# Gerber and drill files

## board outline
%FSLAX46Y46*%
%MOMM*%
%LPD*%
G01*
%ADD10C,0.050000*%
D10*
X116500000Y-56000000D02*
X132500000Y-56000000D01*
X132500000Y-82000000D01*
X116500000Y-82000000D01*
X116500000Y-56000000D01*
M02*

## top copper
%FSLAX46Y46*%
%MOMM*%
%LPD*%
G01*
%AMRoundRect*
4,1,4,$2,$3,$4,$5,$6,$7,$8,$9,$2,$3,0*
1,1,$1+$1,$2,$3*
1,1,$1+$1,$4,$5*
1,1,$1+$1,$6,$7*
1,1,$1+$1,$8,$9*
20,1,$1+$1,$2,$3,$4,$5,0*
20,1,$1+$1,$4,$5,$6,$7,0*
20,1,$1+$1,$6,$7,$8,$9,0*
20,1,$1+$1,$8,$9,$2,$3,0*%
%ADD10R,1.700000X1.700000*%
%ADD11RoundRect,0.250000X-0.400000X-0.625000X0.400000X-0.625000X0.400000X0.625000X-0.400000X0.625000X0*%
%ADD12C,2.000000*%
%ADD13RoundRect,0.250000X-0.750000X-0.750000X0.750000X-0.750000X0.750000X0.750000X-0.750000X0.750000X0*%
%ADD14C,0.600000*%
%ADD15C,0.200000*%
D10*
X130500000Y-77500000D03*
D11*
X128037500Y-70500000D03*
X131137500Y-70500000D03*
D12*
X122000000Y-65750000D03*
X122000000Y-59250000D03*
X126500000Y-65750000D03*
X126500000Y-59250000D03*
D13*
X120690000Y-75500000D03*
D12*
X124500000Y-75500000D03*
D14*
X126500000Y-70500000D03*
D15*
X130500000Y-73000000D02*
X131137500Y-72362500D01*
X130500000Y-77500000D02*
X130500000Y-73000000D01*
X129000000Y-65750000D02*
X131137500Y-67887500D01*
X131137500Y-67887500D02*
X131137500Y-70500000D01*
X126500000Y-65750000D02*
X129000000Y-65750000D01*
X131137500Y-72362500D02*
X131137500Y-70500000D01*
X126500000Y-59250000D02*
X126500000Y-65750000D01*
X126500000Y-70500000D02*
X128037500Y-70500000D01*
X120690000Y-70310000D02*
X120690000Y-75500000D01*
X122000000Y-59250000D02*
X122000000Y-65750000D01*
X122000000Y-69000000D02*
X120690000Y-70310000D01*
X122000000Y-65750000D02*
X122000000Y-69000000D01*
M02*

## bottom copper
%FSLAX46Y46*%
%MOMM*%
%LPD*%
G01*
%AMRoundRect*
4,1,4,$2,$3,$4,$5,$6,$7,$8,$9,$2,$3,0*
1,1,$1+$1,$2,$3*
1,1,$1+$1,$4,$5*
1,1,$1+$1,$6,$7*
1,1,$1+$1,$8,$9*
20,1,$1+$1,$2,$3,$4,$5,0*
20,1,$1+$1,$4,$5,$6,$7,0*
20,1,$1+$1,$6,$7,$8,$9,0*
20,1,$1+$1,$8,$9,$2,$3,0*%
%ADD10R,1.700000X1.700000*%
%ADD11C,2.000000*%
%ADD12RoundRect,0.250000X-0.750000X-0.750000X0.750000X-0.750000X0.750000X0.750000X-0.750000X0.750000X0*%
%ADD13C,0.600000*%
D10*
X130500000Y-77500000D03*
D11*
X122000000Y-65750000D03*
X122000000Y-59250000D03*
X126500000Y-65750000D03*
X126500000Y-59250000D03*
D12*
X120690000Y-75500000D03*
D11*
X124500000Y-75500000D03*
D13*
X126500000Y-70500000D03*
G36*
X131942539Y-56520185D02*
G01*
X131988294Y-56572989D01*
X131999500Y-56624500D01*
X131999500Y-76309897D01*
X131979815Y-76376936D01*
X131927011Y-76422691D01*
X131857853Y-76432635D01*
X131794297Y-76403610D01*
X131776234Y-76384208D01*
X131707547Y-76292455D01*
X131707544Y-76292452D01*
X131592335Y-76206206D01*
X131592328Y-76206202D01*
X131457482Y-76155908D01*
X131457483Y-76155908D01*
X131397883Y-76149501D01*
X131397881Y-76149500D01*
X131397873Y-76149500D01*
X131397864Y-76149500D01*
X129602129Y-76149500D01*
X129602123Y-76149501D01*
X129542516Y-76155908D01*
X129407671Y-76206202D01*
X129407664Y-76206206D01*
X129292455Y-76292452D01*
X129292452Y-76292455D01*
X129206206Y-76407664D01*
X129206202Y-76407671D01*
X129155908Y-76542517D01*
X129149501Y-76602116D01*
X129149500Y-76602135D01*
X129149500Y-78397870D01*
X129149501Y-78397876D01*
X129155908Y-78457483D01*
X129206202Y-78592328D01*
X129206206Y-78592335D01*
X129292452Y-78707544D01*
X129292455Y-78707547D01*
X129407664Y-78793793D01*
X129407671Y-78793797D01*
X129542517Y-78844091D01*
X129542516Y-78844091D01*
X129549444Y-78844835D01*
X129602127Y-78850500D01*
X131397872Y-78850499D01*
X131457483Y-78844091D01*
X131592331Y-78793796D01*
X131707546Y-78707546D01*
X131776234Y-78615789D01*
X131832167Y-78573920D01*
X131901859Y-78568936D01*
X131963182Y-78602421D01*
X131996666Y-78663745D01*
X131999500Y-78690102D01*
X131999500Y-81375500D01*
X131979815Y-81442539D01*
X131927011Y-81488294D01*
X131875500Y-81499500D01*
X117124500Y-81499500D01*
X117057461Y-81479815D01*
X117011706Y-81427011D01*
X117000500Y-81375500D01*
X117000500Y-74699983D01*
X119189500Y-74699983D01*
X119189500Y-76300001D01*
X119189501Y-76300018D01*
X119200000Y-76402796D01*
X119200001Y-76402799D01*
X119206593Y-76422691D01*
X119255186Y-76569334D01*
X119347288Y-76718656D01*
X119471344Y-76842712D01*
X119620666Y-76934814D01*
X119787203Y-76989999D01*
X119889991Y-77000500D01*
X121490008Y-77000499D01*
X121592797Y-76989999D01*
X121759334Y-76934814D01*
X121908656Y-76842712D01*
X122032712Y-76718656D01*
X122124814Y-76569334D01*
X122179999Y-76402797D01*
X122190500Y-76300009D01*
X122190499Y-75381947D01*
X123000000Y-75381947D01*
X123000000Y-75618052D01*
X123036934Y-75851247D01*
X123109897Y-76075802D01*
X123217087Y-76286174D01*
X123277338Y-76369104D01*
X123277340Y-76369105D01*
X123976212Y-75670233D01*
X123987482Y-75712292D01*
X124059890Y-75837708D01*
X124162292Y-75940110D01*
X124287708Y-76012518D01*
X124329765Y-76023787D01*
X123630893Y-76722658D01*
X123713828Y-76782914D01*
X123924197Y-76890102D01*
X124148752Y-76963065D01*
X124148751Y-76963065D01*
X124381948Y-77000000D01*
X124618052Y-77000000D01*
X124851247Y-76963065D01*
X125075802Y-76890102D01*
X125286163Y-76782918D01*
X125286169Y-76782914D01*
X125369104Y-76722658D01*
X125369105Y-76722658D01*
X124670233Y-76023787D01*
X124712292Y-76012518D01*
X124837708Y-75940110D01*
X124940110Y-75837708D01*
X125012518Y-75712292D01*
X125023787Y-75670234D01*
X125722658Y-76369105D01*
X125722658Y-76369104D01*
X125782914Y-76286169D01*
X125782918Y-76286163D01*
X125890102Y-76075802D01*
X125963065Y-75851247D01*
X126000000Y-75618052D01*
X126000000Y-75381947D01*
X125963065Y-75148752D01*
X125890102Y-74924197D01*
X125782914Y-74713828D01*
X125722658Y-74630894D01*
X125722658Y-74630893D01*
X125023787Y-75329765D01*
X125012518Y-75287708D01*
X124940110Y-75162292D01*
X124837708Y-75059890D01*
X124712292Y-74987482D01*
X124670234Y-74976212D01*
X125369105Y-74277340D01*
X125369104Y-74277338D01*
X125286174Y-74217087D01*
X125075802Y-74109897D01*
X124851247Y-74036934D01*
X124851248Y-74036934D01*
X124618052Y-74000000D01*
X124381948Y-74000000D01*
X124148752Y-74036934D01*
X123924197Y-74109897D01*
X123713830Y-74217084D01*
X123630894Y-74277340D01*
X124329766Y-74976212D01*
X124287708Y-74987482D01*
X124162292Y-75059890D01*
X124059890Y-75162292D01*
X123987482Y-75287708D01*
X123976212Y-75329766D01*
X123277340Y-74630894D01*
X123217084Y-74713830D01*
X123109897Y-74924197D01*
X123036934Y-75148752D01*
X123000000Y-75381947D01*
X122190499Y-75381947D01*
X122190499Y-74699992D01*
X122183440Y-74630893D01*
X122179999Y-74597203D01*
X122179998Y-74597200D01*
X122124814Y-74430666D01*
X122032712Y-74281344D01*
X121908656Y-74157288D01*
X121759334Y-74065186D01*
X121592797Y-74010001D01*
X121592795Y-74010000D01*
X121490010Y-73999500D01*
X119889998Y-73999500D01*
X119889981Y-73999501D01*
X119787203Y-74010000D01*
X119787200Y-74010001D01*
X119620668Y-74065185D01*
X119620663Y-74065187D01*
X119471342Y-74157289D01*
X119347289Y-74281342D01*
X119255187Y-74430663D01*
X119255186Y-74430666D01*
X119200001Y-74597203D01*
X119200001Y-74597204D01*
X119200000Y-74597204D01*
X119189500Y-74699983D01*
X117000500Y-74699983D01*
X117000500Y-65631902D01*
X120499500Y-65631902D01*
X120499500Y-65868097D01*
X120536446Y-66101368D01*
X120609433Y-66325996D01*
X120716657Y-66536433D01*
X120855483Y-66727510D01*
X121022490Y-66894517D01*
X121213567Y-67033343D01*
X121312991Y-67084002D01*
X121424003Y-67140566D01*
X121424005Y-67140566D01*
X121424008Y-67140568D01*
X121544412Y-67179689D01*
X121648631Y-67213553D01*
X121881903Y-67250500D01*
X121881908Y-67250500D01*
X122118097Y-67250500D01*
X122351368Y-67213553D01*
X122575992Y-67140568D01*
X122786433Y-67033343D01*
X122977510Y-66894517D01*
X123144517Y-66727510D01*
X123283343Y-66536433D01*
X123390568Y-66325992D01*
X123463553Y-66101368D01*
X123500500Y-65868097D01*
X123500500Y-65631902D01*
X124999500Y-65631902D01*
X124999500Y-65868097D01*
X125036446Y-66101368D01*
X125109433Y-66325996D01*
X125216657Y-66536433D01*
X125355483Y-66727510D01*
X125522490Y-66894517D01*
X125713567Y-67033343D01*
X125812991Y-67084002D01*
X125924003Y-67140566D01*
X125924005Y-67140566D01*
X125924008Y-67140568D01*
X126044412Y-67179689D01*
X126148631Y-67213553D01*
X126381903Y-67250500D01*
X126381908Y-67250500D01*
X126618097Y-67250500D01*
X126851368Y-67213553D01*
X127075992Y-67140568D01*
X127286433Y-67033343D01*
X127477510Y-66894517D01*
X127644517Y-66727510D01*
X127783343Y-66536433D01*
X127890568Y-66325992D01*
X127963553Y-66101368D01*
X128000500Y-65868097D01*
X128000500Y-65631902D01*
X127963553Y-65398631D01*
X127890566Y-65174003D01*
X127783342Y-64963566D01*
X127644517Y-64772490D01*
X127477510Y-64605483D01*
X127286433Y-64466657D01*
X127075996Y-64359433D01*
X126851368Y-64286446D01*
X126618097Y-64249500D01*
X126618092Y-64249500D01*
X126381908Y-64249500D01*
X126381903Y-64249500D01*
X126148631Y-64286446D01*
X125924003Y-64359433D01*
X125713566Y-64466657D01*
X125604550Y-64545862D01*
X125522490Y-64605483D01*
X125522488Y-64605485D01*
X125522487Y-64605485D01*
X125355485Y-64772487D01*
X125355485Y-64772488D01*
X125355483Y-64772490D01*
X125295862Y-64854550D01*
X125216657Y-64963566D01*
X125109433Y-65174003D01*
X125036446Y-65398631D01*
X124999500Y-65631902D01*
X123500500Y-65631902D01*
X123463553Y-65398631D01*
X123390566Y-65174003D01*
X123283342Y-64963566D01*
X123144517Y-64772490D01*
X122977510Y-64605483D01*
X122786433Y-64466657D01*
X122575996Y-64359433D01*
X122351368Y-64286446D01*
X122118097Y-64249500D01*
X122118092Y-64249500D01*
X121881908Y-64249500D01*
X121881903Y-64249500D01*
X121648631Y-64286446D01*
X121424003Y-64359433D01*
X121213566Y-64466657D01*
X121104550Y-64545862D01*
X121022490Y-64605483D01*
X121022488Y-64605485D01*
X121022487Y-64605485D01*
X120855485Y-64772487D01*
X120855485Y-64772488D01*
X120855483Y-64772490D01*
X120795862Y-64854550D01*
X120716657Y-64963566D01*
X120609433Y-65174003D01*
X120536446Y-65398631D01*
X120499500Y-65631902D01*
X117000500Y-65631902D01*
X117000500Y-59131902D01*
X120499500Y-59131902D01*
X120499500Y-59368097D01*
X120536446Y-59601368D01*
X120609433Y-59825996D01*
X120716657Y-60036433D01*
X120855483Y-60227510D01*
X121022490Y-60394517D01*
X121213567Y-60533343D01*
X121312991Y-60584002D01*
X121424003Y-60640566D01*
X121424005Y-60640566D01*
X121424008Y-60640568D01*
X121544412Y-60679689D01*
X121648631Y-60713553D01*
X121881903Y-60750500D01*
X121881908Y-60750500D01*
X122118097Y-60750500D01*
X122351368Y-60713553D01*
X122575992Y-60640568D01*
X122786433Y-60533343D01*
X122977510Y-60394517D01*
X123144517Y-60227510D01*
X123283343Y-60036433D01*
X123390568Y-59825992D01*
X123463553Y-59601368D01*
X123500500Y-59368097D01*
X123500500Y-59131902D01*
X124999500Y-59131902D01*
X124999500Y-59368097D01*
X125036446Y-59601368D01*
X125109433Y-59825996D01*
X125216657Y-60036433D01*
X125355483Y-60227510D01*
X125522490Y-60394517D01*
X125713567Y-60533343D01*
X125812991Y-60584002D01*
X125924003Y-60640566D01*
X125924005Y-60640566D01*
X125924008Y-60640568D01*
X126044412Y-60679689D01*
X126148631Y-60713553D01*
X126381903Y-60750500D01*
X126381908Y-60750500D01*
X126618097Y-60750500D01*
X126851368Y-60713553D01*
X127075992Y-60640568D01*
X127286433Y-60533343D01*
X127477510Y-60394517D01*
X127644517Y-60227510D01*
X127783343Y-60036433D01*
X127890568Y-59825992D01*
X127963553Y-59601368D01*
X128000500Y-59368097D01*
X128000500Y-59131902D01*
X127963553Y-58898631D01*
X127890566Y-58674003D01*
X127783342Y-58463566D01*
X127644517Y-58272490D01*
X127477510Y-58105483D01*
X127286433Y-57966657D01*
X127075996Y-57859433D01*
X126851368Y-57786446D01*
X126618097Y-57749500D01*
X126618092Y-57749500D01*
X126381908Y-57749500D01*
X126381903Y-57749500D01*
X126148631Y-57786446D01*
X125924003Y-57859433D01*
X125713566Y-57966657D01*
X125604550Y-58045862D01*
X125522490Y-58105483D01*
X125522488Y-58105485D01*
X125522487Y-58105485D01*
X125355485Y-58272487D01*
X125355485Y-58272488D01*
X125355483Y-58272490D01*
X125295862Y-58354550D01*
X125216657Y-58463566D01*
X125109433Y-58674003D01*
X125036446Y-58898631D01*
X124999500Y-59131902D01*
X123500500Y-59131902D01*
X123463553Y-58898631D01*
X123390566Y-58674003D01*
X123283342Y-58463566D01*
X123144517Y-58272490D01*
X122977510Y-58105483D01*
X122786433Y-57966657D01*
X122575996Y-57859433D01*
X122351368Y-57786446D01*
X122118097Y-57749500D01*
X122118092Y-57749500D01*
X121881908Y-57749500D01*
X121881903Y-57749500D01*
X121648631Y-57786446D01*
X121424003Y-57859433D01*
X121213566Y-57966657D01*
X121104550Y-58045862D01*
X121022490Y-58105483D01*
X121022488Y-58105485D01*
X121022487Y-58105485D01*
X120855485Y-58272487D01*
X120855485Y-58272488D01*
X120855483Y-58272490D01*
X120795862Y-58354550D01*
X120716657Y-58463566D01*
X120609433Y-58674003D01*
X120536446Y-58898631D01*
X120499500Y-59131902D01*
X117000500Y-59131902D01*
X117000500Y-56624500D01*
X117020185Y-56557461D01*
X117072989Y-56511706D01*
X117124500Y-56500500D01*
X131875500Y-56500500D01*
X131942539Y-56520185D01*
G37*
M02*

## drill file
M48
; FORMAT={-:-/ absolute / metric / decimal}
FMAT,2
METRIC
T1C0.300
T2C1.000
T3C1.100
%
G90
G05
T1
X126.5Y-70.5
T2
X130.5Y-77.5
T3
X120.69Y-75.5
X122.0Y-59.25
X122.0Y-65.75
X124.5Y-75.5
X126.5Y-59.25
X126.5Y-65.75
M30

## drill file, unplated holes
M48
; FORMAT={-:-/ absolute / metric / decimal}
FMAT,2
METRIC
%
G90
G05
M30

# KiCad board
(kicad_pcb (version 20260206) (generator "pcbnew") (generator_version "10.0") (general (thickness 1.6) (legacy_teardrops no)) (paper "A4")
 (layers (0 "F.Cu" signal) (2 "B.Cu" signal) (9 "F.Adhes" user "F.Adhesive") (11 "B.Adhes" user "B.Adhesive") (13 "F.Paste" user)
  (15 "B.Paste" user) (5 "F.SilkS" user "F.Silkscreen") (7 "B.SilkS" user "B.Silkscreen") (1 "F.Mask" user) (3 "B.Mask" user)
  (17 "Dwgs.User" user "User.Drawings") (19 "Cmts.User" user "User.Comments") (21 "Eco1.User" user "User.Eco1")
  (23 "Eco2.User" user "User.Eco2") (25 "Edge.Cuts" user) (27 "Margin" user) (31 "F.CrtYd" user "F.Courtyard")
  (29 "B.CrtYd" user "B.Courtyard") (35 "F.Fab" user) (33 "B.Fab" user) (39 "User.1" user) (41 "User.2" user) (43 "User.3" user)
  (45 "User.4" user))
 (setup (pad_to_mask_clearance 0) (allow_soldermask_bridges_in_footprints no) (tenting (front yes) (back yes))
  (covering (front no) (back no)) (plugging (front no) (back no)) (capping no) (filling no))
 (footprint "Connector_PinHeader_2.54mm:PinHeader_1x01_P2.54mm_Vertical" (layer "F.Cu") (at 130.5 77.5)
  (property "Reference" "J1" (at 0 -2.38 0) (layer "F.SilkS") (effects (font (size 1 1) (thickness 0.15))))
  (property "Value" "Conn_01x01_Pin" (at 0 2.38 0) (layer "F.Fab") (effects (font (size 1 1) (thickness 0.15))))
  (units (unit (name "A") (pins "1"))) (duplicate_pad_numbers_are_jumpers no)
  (pad "1" thru_hole rect (at 0 0) (size 1.7 1.7) (drill 1) (layers "*.Cu" "*.Mask") (remove_unused_layers no) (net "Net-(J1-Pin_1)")))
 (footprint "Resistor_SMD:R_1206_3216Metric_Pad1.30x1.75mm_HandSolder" (layer "F.Cu") (at 129.5875 70.5)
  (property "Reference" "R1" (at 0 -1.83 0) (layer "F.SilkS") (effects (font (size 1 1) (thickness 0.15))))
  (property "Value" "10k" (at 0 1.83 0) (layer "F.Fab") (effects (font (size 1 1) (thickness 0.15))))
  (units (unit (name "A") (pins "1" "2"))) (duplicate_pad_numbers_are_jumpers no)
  (pad "1" smd roundrect (at -1.55 0) (size 1.3 1.75) (layers "F.Cu" "F.Mask" "F.Paste") (roundrect_rratio 0.192308) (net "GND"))
  (pad "2" smd roundrect (at 1.55 0) (size 1.3 1.75) (layers "F.Cu" "F.Mask" "F.Paste") (roundrect_rratio 0.192308) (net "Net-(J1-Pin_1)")))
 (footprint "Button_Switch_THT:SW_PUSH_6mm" (layer "F.Cu") (at 122 65.75 90)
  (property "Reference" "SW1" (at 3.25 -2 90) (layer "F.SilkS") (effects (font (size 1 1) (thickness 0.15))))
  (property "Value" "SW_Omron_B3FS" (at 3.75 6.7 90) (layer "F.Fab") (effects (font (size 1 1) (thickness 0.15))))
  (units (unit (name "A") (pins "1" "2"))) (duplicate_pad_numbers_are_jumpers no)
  (pad "1" thru_hole circle (at 0 0 180) (size 2 2) (drill 1.1) (layers "*.Cu" "*.Mask") (remove_unused_layers no) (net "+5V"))
  (pad "1" thru_hole circle (at 6.5 0 180) (size 2 2) (drill 1.1) (layers "*.Cu" "*.Mask") (remove_unused_layers no) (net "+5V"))
  (pad "2" thru_hole circle (at 0 4.5 180) (size 2 2) (drill 1.1) (layers "*.Cu" "*.Mask") (remove_unused_layers no) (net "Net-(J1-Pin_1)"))
  (pad "2" thru_hole circle (at 6.5 4.5 180) (size 2 2) (drill 1.1) (layers "*.Cu" "*.Mask") (remove_unused_layers no)
   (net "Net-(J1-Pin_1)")))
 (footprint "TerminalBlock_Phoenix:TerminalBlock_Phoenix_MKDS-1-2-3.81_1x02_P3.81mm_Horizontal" (layer "F.Cu") (at 120.69 75.5)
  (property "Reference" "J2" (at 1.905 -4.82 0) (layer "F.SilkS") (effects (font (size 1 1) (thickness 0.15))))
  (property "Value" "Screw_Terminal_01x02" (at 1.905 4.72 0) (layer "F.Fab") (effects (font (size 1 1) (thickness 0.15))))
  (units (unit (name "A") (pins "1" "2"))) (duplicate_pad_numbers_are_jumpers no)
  (pad "1" thru_hole roundrect (at 0 0) (size 2 2) (drill 1.1) (layers "*.Cu" "*.Mask") (remove_unused_layers no) (roundrect_rratio 0.125)
   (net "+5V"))
  (pad "2" thru_hole circle (at 3.81 0) (size 2 2) (drill 1.1) (layers "*.Cu" "*.Mask") (remove_unused_layers no) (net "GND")))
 (gr_rect (start 116.5 56) (end 132.5 82) (stroke (width 0.05) (type default)) (fill no) (layer "Edge.Cuts"))
 (segment (start 130.5 73) (end 131.1375 72.3625) (width 0.2) (layer "F.Cu") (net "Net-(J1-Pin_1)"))
 (segment (start 130.5 77.5) (end 130.5 73) (width 0.2) (layer "F.Cu") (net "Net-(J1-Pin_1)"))
 (segment (start 129 65.75) (end 131.1375 67.8875) (width 0.2) (layer "F.Cu") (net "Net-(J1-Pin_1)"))
 (segment (start 131.1375 67.8875) (end 131.1375 70.5) (width 0.2) (layer "F.Cu") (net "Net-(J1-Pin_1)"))
 (segment (start 126.5 65.75) (end 129 65.75) (width 0.2) (layer "F.Cu") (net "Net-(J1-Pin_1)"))
 (segment (start 131.1375 72.3625) (end 131.1375 70.5) (width 0.2) (layer "F.Cu") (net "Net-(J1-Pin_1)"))
 (segment (start 126.5 59.25) (end 126.5 65.75) (width 0.2) (layer "F.Cu") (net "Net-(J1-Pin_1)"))
 (segment (start 126.5 70.5) (end 128.0375 70.5) (width 0.2) (layer "F.Cu") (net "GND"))
 (via (at 126.5 70.5) (size 0.6) (drill 0.3) (layers "F.Cu" "B.Cu") (free yes) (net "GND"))
 (segment (start 120.69 70.31) (end 120.69 75.5) (width 0.2) (layer "F.Cu") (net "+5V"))
 (segment (start 122 59.25) (end 122 65.75) (width 0.2) (layer "F.Cu") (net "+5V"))
 (segment (start 122 69) (end 120.69 70.31) (width 0.2) (layer "F.Cu") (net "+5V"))
 (segment (start 122 65.75) (end 122 69) (width 0.2) (layer "F.Cu") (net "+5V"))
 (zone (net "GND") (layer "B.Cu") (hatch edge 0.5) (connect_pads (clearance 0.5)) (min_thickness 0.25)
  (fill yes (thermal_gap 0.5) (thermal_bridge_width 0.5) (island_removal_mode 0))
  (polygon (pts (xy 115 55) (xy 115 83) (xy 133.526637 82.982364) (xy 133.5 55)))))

